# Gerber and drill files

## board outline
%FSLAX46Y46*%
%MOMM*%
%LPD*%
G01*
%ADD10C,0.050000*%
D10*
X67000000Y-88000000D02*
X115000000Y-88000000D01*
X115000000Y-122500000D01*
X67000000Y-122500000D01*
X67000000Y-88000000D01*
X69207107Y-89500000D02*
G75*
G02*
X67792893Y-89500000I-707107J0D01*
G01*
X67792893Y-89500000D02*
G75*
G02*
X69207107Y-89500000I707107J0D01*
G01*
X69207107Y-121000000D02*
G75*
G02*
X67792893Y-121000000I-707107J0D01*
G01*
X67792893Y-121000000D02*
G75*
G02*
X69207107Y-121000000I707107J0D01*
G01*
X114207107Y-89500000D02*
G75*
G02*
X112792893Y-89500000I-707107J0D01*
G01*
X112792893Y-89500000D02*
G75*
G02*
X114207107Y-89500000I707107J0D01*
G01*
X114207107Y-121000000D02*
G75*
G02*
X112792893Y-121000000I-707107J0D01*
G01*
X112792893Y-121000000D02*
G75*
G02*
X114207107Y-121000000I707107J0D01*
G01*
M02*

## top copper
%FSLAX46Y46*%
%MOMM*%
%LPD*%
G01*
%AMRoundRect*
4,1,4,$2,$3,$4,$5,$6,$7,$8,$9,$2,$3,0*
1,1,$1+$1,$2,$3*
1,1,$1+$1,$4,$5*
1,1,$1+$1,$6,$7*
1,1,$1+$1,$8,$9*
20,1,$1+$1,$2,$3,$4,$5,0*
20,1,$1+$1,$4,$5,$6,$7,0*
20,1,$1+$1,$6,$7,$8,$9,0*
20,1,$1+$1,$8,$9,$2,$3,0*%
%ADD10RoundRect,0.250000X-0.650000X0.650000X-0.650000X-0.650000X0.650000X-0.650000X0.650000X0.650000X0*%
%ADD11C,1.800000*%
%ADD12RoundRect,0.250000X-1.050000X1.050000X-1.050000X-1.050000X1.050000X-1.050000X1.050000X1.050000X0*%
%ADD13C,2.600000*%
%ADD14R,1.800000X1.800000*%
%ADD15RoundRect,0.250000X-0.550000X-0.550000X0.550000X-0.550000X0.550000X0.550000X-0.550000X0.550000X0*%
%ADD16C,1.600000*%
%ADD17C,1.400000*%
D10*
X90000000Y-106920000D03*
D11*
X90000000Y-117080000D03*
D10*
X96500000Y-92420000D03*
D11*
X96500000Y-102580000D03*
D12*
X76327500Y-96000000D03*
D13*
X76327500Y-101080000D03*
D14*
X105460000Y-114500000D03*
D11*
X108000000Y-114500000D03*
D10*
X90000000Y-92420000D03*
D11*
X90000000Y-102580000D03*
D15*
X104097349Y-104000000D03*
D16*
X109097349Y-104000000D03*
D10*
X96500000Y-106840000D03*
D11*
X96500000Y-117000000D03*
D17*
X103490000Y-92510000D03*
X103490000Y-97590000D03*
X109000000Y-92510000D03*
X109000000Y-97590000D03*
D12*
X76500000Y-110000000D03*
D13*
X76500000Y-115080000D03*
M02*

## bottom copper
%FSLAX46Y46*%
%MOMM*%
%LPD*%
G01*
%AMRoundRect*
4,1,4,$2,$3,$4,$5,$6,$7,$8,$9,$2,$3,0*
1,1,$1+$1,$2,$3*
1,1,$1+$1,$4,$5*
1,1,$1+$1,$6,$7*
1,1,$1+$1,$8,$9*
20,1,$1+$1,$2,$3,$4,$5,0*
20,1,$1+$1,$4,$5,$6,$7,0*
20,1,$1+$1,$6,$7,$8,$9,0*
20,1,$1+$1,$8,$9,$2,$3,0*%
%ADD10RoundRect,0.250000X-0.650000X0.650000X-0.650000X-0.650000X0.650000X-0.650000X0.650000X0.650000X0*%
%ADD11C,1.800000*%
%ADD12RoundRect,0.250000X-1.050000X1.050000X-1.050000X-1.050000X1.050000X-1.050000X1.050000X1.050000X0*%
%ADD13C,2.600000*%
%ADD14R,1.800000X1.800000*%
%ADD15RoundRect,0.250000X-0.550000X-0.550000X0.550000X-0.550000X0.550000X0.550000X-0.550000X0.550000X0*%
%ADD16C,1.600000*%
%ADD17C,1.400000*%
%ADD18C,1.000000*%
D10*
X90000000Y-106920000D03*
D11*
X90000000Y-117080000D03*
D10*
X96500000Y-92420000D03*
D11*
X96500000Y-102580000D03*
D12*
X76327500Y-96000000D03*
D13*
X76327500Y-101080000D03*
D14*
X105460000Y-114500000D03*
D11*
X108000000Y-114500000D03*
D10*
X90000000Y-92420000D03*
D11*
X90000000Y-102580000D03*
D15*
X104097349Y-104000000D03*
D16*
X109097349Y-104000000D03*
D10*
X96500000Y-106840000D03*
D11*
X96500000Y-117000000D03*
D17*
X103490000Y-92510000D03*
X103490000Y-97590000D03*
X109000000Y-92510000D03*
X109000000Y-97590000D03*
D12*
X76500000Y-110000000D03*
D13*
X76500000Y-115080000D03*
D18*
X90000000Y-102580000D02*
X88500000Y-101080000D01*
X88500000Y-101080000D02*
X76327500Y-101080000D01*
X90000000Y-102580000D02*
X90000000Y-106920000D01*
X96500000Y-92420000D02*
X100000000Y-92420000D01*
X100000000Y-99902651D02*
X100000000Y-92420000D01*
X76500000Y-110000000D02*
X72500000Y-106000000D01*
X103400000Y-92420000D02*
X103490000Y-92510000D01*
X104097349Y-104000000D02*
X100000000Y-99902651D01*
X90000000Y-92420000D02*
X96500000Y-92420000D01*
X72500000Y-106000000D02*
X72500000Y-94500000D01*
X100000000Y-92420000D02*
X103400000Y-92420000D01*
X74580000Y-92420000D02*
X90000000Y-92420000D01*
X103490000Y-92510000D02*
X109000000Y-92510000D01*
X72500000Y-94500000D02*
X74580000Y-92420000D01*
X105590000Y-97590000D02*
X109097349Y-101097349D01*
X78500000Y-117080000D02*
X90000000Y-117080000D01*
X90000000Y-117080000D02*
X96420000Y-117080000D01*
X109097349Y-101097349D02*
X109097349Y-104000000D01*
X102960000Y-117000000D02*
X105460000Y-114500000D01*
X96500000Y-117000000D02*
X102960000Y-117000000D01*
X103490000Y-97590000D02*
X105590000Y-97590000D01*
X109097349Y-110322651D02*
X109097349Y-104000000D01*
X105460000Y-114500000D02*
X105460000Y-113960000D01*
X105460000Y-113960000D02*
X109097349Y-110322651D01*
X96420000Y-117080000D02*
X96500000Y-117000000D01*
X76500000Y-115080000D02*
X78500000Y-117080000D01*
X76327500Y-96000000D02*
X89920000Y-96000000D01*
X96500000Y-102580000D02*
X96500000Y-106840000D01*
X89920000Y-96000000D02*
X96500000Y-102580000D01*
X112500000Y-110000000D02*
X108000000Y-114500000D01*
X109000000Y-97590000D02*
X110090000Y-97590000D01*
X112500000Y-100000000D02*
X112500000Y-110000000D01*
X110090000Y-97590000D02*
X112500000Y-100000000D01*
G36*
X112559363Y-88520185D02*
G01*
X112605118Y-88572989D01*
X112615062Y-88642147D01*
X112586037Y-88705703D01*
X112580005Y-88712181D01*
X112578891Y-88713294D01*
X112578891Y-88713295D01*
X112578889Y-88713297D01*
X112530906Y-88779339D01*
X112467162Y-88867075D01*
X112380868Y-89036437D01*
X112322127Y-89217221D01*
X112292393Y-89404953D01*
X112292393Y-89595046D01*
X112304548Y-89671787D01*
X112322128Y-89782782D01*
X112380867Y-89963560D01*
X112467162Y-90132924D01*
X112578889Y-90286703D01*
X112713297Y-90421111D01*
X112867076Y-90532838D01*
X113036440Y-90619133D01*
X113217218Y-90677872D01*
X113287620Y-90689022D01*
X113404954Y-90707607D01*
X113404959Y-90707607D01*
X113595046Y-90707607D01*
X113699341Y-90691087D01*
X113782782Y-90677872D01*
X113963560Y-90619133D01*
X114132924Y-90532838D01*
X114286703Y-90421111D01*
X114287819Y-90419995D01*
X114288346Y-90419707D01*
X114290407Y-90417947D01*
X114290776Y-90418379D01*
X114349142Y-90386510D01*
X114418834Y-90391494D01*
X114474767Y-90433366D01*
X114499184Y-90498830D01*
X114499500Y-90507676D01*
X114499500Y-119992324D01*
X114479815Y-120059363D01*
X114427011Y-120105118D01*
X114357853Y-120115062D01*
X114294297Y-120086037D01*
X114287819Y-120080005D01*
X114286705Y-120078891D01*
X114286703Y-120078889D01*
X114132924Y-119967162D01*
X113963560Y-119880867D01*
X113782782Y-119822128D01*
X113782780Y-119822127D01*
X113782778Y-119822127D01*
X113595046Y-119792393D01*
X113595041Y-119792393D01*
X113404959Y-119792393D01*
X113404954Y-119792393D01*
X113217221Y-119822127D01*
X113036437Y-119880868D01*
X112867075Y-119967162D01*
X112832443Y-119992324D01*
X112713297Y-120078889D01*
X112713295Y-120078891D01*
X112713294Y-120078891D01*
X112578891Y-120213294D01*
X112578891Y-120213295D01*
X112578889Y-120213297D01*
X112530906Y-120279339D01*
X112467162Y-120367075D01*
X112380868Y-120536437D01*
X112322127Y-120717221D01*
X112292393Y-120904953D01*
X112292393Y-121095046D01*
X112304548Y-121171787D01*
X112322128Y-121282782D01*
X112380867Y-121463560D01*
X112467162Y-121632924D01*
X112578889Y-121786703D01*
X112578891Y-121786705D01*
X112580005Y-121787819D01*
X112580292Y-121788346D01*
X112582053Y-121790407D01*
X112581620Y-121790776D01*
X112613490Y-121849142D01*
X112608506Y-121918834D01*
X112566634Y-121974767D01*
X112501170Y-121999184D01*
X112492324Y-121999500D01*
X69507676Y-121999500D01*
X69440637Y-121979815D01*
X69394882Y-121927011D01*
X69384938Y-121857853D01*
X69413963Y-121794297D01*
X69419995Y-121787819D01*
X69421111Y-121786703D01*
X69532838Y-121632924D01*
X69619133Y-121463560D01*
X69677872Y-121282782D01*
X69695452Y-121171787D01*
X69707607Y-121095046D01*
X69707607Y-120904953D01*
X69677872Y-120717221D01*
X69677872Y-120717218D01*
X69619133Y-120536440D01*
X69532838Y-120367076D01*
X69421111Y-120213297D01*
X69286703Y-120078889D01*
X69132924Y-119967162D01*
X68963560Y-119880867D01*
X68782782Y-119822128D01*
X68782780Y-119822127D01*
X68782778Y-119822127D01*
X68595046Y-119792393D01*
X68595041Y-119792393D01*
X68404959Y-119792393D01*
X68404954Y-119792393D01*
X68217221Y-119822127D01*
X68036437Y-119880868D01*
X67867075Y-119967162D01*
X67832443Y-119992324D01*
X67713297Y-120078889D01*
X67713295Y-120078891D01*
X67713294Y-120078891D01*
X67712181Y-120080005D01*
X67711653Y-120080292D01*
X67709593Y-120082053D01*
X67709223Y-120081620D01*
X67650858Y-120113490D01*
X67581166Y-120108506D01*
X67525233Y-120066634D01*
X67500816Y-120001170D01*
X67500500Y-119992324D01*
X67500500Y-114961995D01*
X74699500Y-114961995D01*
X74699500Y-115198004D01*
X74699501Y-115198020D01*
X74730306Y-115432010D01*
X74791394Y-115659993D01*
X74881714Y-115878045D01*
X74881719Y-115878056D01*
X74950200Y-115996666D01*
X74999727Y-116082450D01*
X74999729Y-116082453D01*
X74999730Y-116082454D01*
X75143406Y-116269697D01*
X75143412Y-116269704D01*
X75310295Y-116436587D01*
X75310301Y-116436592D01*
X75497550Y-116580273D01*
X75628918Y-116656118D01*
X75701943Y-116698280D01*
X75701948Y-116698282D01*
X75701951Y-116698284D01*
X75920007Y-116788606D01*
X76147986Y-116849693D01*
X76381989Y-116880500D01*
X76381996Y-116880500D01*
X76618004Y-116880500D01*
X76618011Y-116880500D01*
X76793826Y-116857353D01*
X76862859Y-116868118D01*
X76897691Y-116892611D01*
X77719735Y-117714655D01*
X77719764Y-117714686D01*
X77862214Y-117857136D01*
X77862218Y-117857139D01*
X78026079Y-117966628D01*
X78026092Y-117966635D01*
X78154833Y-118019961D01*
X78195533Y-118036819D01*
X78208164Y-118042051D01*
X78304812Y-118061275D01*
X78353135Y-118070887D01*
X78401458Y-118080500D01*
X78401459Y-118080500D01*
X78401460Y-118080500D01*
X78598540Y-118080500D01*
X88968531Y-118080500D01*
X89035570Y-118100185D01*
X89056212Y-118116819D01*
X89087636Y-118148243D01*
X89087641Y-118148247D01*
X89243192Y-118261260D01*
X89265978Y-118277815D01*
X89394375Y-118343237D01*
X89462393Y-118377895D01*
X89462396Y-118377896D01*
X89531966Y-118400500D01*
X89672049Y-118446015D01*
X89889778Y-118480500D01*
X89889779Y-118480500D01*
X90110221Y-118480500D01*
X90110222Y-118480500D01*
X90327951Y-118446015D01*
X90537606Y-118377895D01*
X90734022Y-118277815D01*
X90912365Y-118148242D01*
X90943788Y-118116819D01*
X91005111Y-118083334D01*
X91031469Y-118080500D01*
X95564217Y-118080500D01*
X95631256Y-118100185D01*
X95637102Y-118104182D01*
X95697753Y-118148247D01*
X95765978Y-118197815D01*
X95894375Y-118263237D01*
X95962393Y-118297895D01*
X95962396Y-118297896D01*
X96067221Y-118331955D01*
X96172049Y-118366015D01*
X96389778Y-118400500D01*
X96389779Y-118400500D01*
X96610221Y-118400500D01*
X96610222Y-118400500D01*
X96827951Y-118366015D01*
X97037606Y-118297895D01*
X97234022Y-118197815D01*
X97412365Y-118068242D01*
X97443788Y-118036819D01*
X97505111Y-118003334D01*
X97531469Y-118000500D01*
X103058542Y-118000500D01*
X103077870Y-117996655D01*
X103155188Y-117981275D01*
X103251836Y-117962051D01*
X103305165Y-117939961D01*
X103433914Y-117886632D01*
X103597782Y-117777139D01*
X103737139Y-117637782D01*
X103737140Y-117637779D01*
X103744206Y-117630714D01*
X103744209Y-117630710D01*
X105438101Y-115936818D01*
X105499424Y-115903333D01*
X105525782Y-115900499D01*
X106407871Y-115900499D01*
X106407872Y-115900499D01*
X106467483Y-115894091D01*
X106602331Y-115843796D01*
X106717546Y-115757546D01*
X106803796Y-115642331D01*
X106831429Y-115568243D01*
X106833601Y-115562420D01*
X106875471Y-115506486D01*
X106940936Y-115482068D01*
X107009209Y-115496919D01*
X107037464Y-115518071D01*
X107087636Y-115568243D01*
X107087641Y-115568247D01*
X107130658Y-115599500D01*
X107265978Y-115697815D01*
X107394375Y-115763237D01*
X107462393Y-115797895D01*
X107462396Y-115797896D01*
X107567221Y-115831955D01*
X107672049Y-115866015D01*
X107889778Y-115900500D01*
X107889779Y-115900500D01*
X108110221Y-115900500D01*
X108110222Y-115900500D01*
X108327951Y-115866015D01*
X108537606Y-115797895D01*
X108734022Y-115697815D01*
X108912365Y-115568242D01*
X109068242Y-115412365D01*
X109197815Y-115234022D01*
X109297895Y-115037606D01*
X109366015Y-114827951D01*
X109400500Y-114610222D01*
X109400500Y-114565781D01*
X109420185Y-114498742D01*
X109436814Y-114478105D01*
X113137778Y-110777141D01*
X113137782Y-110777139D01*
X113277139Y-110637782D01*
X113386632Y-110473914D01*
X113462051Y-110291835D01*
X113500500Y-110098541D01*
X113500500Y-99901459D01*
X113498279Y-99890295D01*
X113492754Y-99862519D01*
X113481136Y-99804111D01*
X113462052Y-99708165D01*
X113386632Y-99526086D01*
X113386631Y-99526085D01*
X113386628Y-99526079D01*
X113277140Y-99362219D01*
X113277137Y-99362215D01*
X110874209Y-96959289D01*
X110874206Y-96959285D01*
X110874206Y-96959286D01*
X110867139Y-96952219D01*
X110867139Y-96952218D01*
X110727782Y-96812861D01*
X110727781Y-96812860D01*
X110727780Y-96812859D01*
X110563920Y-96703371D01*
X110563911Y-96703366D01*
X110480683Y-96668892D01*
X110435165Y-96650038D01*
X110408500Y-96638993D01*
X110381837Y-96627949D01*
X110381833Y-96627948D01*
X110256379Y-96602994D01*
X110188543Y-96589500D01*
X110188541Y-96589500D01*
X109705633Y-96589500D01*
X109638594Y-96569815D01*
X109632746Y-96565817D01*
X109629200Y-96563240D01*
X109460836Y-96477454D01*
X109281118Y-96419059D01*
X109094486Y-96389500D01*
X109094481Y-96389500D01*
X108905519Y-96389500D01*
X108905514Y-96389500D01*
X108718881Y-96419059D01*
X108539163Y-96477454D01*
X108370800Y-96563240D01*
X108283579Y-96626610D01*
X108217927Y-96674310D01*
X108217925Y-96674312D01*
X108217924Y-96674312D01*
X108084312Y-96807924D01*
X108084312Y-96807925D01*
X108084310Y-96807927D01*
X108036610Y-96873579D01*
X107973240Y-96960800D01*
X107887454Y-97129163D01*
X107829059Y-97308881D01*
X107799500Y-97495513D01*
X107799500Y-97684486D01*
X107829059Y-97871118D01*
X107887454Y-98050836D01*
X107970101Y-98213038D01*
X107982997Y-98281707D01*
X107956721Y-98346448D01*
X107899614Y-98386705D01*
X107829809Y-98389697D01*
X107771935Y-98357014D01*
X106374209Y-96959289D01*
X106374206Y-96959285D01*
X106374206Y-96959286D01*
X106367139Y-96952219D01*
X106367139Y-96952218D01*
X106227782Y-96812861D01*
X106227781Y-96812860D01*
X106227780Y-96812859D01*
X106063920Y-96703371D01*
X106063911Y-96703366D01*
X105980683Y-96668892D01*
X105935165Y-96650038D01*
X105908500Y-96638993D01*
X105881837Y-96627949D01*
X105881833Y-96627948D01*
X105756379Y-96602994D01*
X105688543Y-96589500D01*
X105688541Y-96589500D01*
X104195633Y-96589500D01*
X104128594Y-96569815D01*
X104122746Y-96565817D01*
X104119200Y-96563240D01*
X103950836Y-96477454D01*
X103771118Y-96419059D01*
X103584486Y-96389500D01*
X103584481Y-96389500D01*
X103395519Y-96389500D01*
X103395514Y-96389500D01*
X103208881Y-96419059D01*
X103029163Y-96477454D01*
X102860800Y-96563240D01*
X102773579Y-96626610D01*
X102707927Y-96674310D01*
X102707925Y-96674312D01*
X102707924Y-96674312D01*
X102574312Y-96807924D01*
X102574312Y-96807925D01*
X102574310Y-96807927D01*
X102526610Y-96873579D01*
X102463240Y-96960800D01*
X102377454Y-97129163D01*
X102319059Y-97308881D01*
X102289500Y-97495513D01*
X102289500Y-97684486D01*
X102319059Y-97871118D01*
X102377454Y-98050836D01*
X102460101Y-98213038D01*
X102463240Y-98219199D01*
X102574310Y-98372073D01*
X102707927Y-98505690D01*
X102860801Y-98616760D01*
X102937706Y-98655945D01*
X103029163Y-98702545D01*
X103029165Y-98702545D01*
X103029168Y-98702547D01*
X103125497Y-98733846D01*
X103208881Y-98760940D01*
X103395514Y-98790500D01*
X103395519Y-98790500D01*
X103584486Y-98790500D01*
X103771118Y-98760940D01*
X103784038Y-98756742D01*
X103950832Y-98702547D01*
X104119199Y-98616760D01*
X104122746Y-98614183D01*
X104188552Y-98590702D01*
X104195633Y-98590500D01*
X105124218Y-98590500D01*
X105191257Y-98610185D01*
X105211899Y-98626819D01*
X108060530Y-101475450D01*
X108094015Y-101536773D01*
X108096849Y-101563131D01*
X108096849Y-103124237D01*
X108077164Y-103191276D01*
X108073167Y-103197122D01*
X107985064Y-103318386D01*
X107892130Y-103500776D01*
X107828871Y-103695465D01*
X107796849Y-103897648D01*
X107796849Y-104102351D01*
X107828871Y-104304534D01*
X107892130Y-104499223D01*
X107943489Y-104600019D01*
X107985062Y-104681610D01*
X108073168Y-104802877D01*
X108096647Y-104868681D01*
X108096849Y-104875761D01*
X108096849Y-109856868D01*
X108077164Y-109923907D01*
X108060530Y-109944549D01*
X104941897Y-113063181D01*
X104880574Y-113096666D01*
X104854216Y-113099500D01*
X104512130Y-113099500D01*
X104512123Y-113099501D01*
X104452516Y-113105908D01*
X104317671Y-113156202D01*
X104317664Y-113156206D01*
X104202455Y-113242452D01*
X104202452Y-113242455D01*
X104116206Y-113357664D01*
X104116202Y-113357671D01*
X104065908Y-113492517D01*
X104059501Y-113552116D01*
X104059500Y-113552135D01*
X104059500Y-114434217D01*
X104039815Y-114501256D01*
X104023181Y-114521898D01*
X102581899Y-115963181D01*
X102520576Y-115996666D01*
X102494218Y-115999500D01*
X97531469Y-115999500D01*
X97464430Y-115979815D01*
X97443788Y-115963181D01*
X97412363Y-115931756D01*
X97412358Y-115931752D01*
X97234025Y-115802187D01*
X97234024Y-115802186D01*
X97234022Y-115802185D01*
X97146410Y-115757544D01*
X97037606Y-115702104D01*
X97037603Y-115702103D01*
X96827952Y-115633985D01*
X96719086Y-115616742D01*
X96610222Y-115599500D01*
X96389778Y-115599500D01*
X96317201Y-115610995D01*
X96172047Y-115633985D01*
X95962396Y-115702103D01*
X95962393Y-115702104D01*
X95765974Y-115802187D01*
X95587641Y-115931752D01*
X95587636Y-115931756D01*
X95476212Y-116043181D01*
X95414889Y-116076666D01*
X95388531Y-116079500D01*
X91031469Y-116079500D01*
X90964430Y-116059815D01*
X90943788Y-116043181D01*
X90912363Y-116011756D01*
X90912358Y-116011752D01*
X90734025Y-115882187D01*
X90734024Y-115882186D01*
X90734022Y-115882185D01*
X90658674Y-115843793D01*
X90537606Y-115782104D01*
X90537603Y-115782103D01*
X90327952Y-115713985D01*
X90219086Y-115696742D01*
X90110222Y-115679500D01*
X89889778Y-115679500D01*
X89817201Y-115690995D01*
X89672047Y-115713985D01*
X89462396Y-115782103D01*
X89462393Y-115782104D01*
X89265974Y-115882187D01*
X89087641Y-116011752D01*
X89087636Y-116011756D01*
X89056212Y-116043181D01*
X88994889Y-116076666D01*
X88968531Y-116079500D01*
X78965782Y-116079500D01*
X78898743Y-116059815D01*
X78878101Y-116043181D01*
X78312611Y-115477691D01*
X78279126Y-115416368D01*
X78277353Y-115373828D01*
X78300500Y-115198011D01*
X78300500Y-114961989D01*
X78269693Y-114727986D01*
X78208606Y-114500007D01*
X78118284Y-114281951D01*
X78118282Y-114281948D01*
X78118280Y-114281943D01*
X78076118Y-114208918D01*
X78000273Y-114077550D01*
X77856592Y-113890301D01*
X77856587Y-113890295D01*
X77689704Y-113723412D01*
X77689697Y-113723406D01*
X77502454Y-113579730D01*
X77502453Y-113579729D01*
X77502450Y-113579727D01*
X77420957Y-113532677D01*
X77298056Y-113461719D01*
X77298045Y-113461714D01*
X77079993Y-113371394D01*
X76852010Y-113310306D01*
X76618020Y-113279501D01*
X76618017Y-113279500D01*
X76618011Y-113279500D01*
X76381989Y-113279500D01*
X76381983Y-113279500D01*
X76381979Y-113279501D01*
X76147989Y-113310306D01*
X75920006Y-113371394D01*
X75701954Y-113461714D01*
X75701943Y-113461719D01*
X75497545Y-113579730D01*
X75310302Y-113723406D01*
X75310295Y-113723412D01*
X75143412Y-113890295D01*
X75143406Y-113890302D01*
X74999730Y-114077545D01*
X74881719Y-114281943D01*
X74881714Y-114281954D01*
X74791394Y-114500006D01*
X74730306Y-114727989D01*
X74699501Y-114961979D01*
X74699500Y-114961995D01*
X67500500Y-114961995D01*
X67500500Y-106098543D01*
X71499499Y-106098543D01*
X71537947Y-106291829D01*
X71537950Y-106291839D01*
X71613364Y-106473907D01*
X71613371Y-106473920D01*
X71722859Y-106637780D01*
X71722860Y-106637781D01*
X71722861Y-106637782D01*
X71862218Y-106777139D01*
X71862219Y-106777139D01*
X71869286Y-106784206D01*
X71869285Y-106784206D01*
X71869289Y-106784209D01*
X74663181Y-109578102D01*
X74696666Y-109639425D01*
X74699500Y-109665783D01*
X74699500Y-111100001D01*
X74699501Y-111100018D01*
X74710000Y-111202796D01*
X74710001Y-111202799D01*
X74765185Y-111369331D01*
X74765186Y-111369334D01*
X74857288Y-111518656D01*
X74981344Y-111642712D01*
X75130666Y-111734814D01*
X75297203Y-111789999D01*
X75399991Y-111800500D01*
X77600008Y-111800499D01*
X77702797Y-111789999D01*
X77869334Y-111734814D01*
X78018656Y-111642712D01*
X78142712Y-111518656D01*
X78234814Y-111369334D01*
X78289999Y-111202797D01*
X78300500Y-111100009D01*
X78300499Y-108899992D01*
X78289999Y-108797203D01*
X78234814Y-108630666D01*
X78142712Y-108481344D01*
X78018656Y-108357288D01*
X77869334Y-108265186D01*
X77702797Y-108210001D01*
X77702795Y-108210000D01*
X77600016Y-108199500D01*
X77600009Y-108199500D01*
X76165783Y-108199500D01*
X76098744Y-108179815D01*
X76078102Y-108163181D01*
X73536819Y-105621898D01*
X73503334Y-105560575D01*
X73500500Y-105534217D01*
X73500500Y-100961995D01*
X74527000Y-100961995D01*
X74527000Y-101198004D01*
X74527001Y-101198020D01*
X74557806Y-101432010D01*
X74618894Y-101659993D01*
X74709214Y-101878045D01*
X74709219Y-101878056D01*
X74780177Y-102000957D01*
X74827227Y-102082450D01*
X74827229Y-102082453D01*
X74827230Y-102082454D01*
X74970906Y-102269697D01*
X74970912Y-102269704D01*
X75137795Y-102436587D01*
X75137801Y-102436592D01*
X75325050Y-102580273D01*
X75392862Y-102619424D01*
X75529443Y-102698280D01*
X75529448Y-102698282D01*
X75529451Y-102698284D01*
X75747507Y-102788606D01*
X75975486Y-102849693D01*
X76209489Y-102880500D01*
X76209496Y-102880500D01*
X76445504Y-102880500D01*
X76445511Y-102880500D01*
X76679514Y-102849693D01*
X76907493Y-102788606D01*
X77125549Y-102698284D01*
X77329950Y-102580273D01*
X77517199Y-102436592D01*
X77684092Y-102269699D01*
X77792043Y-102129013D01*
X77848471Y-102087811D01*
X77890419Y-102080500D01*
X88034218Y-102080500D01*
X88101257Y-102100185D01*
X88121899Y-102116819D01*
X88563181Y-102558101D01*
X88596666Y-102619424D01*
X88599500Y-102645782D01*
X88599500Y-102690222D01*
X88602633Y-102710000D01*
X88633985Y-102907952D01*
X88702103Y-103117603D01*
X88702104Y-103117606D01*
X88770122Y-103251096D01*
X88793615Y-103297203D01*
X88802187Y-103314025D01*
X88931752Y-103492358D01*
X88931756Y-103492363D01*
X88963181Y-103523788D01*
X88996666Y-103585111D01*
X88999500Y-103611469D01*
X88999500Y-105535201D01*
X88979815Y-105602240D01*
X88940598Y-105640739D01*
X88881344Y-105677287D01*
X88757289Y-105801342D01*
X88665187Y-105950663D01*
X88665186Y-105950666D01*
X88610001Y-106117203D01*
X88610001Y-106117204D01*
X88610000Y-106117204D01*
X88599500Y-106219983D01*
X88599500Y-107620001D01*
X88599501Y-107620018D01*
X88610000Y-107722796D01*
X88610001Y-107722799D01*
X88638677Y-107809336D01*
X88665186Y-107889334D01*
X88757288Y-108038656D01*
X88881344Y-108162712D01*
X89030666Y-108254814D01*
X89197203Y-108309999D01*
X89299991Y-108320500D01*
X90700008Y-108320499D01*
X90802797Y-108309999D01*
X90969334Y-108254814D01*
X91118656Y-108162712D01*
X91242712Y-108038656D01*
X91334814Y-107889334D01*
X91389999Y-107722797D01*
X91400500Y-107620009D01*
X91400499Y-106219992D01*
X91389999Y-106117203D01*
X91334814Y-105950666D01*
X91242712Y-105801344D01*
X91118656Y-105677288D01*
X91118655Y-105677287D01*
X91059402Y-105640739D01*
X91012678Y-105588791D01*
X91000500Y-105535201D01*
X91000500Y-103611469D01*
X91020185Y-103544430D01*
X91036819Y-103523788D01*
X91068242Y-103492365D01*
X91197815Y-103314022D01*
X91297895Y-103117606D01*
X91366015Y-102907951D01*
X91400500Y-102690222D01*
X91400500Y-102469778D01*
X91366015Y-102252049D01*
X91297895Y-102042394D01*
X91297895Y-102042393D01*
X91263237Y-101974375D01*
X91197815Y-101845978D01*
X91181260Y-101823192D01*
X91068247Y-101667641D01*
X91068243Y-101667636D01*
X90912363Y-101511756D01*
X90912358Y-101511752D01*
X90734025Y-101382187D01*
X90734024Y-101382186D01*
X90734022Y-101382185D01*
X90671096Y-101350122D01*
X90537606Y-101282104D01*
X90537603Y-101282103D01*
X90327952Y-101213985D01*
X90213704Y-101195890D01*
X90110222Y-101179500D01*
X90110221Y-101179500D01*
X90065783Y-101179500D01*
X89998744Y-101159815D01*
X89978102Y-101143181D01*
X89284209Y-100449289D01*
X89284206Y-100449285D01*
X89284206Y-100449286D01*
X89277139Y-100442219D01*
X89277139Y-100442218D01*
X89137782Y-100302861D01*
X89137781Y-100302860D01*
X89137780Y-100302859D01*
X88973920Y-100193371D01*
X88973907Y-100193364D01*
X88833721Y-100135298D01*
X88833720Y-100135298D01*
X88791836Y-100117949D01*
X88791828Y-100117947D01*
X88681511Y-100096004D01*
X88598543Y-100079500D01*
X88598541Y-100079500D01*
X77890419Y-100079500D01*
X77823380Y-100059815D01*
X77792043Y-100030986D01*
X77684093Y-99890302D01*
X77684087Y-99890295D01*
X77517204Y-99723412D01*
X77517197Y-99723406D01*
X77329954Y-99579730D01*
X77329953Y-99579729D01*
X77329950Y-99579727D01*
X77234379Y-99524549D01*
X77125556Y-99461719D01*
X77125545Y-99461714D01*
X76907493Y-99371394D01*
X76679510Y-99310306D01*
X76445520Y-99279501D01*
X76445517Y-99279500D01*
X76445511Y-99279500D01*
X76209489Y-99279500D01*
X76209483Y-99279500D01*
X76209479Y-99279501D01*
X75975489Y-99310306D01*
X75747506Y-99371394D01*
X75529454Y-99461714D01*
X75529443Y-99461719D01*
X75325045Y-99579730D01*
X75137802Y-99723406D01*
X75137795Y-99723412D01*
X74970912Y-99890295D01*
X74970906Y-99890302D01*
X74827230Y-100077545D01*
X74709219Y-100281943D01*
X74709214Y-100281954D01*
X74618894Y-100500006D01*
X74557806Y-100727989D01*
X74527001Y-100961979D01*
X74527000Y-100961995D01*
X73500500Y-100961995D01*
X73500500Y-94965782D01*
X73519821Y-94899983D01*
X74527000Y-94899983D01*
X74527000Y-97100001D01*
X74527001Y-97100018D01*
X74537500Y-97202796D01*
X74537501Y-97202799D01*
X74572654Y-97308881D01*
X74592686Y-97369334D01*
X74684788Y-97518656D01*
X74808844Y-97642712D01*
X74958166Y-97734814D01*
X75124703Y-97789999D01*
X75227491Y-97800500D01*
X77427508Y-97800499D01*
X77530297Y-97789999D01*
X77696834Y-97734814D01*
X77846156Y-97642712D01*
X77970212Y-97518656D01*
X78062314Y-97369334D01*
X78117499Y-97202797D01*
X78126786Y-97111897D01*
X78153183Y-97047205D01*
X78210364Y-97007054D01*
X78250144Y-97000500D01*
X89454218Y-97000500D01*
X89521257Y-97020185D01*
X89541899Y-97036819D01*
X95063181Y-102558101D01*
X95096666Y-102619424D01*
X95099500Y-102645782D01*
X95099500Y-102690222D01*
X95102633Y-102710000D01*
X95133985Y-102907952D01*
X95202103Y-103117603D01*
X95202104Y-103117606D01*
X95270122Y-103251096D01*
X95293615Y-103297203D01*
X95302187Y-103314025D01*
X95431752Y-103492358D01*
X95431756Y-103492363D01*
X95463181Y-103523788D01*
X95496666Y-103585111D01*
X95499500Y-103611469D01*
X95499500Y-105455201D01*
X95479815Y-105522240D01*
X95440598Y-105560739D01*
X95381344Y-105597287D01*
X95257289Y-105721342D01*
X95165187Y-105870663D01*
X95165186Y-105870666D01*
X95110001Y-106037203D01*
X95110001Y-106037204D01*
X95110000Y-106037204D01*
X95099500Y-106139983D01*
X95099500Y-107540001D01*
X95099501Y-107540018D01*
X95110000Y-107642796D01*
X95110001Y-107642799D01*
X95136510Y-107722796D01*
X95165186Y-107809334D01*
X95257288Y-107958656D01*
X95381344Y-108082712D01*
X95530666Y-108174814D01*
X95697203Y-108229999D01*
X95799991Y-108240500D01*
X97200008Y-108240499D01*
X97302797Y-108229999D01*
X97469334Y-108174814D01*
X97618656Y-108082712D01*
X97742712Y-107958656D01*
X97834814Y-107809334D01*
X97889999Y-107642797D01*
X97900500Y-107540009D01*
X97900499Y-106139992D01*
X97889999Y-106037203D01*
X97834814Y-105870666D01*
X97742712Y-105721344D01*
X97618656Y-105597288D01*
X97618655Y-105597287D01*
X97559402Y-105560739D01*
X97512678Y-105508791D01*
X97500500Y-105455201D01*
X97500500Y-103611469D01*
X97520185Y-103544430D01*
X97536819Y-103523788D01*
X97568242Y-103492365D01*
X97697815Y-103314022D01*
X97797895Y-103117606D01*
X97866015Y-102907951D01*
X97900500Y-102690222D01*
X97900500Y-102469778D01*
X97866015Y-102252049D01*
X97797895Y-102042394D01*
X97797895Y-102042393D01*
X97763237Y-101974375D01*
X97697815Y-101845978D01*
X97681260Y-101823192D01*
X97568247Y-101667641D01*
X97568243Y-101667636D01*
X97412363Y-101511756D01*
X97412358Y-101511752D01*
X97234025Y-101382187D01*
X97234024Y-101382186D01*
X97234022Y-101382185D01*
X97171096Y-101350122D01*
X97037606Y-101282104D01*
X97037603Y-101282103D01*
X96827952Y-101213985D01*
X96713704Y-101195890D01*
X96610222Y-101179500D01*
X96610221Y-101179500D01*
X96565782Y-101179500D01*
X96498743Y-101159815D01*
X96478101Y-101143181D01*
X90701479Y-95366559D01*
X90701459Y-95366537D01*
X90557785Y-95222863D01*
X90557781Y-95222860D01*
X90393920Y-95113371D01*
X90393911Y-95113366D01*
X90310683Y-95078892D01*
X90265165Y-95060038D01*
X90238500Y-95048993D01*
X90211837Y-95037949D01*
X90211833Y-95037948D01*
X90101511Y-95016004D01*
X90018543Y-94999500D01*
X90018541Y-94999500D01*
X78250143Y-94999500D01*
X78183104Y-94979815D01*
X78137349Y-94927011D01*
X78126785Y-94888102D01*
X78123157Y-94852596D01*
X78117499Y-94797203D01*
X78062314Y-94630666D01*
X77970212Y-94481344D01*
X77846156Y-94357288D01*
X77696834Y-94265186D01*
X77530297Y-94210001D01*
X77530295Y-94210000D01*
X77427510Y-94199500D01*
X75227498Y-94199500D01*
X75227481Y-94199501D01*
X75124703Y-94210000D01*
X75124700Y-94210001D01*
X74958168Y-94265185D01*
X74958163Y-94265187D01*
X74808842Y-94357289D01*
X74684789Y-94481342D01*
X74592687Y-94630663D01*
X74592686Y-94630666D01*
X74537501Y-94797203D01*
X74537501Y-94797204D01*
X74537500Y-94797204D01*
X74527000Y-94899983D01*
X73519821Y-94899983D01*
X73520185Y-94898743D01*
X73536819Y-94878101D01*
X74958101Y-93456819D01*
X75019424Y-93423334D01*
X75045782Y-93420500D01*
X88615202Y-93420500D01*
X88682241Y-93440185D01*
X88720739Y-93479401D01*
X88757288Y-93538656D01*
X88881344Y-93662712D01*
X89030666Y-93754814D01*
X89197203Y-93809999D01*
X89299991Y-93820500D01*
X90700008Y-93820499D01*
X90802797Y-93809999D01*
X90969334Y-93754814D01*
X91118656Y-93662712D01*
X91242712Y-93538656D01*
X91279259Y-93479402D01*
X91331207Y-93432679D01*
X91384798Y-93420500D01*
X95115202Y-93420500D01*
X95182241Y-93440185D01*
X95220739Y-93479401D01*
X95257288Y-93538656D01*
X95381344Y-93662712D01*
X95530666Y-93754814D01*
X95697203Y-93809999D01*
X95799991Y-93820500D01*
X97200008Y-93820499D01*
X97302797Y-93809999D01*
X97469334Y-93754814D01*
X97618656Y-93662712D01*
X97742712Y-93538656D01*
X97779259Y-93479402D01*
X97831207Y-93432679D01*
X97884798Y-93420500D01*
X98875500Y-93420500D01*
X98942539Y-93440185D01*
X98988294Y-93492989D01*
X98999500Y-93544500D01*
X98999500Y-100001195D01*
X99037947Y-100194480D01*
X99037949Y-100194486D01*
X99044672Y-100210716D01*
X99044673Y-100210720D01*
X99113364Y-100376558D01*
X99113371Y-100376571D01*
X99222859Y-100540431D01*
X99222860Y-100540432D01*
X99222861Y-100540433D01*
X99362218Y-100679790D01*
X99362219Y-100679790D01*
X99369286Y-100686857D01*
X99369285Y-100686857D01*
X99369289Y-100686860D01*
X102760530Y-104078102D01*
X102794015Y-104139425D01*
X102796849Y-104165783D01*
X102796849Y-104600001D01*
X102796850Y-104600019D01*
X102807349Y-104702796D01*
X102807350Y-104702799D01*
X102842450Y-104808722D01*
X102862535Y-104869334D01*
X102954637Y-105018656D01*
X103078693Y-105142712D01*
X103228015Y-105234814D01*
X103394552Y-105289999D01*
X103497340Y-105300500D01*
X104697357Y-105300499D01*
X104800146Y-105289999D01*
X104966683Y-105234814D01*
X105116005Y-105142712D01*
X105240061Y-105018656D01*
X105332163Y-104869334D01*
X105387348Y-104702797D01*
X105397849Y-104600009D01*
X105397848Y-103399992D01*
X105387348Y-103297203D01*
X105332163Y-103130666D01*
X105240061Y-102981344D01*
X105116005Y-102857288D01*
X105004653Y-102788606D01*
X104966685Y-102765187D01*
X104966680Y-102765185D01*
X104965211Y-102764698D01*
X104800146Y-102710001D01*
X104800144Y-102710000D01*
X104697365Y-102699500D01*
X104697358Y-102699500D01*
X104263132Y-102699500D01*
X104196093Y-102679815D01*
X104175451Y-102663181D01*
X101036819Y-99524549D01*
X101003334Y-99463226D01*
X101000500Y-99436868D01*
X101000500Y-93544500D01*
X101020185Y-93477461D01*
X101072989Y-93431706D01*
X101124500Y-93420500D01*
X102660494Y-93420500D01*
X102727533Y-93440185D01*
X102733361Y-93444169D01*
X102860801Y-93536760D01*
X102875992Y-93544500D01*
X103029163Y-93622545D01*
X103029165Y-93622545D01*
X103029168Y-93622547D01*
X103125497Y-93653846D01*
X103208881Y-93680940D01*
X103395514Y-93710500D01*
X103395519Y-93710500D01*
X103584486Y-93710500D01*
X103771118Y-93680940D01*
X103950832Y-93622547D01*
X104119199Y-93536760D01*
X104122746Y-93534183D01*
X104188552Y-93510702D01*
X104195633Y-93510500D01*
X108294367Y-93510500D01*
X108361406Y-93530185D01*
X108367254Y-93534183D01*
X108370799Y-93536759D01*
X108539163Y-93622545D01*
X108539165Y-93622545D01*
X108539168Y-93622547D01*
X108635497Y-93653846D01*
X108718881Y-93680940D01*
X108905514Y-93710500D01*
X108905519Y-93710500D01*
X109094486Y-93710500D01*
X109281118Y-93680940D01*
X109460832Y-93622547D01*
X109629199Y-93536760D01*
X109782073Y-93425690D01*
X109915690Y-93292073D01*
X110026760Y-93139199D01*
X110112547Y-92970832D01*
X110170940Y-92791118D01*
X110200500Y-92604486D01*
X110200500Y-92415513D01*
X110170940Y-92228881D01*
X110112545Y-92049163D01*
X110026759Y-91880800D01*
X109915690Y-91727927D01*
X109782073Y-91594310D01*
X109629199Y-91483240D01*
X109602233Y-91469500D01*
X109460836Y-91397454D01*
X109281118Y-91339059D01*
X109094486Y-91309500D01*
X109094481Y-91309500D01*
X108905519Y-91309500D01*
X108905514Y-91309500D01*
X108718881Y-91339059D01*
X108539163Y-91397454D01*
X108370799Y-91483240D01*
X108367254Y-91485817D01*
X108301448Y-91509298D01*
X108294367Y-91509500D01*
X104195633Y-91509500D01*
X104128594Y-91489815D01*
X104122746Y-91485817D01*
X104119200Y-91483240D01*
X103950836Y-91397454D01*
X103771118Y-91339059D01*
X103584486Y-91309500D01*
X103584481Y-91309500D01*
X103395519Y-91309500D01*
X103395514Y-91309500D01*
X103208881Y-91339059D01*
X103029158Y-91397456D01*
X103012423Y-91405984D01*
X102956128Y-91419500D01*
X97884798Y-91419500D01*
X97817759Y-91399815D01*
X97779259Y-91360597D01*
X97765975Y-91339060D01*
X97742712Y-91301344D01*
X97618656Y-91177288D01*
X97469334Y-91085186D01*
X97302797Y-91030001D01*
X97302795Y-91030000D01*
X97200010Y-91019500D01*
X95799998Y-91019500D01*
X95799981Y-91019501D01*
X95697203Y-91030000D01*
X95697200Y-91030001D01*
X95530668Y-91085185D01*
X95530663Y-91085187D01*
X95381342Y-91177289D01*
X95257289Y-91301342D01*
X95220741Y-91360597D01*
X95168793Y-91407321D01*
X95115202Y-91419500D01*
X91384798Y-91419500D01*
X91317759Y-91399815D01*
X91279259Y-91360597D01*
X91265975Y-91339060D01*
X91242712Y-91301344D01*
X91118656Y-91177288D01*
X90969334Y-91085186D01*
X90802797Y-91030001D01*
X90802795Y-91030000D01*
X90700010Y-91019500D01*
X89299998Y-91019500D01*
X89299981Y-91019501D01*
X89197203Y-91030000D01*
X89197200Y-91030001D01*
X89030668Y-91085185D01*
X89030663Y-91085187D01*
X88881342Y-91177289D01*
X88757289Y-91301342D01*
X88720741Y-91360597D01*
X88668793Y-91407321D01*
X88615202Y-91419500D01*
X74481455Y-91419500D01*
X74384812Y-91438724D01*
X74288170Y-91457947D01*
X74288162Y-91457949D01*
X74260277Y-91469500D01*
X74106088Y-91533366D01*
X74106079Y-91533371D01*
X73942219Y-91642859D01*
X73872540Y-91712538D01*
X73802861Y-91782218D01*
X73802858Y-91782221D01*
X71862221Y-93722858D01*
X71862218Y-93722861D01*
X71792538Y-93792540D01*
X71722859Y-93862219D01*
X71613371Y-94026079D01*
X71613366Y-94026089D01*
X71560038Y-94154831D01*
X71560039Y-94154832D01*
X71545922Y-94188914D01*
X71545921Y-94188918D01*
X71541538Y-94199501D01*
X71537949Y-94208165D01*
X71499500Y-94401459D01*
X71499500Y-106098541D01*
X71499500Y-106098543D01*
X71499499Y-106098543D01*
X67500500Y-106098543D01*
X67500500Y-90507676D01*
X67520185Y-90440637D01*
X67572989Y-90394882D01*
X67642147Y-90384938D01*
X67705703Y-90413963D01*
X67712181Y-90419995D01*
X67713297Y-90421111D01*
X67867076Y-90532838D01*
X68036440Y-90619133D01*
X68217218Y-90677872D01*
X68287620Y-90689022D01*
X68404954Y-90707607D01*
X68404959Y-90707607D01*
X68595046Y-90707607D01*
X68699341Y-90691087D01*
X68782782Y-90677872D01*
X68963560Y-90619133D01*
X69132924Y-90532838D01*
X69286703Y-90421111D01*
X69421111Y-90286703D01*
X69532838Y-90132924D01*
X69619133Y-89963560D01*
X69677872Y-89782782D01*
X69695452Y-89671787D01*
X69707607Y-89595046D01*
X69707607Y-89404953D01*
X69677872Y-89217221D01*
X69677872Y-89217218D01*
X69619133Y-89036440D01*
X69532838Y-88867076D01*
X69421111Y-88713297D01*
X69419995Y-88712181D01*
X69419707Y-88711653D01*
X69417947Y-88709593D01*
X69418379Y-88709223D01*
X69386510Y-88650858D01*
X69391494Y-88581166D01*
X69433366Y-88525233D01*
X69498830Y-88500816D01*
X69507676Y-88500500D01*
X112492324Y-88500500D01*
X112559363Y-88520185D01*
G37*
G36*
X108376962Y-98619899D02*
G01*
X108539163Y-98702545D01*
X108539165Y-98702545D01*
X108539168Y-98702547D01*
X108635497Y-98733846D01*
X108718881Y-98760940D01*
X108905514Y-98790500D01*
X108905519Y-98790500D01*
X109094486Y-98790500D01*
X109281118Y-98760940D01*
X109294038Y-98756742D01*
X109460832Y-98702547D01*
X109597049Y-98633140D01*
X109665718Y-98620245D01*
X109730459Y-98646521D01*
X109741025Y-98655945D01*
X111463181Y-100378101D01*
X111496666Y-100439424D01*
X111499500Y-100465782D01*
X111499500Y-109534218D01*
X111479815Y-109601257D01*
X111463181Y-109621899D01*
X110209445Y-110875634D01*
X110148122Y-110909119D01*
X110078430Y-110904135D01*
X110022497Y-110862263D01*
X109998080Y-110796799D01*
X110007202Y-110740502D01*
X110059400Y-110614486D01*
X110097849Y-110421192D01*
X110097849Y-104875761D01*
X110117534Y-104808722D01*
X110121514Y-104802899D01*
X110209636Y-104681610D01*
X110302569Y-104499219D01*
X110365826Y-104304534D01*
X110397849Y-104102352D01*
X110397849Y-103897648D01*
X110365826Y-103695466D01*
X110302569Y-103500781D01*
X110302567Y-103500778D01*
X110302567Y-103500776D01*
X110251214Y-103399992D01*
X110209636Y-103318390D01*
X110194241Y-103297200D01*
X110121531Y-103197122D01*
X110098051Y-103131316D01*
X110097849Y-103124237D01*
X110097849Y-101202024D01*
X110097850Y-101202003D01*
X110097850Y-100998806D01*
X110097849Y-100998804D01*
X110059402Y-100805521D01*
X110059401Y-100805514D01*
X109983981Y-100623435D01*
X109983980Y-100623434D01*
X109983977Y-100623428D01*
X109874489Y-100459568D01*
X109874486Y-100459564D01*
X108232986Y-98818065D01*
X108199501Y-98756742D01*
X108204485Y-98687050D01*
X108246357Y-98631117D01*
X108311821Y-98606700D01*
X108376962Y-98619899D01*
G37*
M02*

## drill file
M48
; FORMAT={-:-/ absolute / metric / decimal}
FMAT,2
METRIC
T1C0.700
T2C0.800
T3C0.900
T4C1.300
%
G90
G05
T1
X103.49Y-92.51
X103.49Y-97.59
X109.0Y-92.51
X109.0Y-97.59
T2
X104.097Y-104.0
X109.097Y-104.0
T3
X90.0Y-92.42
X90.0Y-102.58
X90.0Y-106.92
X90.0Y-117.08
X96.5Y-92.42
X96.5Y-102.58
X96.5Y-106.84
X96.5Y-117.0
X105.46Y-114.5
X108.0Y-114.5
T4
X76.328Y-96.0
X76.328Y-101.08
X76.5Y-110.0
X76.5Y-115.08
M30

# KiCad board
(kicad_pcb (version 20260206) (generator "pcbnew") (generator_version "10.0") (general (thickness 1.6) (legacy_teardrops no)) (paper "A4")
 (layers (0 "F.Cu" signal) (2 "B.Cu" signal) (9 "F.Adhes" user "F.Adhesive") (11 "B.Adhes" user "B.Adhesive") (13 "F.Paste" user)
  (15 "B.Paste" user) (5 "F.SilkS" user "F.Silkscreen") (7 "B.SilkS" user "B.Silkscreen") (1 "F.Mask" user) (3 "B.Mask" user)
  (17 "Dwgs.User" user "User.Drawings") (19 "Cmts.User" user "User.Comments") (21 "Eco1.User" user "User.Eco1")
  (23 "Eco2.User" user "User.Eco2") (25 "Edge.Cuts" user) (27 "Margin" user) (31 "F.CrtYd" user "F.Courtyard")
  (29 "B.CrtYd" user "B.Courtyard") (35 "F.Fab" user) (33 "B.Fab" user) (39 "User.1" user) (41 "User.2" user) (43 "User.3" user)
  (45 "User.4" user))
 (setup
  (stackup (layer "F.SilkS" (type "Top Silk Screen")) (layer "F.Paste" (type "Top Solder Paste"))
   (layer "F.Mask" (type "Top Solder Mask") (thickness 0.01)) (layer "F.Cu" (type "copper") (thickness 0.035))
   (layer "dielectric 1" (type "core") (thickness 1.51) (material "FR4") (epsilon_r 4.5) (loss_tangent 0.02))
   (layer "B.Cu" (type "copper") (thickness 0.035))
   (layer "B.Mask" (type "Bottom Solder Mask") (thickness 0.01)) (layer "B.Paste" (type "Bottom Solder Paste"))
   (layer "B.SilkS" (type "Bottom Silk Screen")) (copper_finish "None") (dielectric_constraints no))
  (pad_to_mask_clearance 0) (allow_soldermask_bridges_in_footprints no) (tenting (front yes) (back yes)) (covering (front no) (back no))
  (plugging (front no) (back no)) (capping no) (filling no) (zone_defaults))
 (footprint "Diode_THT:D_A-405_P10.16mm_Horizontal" (layer "F.Cu") (at 90 106.92 -90)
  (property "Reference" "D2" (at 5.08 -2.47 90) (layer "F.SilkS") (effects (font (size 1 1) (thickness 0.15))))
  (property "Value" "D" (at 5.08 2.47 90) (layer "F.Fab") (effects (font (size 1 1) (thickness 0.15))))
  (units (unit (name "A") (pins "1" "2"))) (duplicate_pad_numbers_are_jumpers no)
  (pad "1" thru_hole roundrect (at 0 0 270) (size 1.8 1.8) (drill 0.9) (layers "*.Cu" "*.Mask") (remove_unused_layers no)
   (roundrect_rratio 0.138889) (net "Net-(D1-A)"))
  (pad "2" thru_hole circle (at 10.16 0 270) (size 1.8 1.8) (drill 0.9) (layers "*.Cu" "*.Mask") (remove_unused_layers no)
   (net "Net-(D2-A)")))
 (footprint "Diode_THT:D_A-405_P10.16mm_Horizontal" (layer "F.Cu") (at 96.5 92.42 -90)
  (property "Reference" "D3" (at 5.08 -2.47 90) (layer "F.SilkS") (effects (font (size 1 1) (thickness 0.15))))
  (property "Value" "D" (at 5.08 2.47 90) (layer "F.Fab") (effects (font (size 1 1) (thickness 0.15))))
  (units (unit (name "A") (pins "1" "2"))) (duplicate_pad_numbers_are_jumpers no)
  (pad "1" thru_hole roundrect (at 0 0 270) (size 1.8 1.8) (drill 0.9) (layers "*.Cu" "*.Mask") (remove_unused_layers no)
   (roundrect_rratio 0.138889) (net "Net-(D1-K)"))
  (pad "2" thru_hole circle (at 10.16 0 270) (size 1.8 1.8) (drill 0.9) (layers "*.Cu" "*.Mask") (remove_unused_layers no)
   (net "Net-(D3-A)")))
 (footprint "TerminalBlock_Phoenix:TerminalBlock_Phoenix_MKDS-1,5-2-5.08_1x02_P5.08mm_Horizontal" (layer "F.Cu") (at 76.3275 96 -90)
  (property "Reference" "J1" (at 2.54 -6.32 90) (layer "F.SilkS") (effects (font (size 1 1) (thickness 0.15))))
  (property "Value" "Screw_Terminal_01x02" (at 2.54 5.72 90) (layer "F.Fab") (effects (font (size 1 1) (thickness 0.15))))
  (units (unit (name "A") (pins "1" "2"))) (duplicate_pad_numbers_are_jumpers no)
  (pad "1" thru_hole roundrect (at 0 0 270) (size 2.6 2.6) (drill 1.3) (layers "*.Cu" "*.Mask") (remove_unused_layers no)
   (roundrect_rratio 0.096154) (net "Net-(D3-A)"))
  (pad "2" thru_hole circle (at 5.08 0 270) (size 2.6 2.6) (drill 1.3) (layers "*.Cu" "*.Mask") (remove_unused_layers no) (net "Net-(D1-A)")))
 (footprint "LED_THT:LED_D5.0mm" (layer "F.Cu") (at 105.46 114.5)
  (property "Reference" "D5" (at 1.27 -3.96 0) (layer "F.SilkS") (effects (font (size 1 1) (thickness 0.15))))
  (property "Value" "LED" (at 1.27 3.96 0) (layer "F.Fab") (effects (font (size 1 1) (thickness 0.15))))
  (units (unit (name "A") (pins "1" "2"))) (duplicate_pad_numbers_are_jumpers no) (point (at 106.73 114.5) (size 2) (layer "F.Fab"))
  (pad "1" thru_hole rect (at 0 0) (size 1.8 1.8) (drill 0.9) (layers "*.Cu" "*.Mask") (remove_unused_layers no) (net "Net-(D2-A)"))
  (pad "2" thru_hole circle (at 2.54 0) (size 1.8 1.8) (drill 0.9) (layers "*.Cu" "*.Mask") (remove_unused_layers no) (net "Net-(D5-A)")))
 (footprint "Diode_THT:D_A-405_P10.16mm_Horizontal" (layer "F.Cu") (at 90 92.42 -90)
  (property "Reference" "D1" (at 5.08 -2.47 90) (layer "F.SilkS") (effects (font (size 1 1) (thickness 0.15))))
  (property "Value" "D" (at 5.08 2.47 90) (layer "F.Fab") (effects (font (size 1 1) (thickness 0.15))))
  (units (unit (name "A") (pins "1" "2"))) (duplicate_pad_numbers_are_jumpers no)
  (pad "1" thru_hole roundrect (at 0 0 270) (size 1.8 1.8) (drill 0.9) (layers "*.Cu" "*.Mask") (remove_unused_layers no)
   (roundrect_rratio 0.138889) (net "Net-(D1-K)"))
  (pad "2" thru_hole circle (at 10.16 0 270) (size 1.8 1.8) (drill 0.9) (layers "*.Cu" "*.Mask") (remove_unused_layers no)
   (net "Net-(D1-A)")))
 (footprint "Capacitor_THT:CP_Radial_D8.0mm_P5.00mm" (layer "F.Cu") (at 104.097349 104)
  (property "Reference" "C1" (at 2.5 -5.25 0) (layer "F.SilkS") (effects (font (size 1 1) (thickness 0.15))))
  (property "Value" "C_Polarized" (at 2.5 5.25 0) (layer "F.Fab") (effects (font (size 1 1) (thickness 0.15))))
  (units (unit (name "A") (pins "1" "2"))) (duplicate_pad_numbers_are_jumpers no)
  (pad "1" thru_hole roundrect (at 0 0) (size 1.6 1.6) (drill 0.8) (layers "*.Cu" "*.Mask") (remove_unused_layers no)
   (roundrect_rratio 0.15625) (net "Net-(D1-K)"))
  (pad "2" thru_hole circle (at 5 0) (size 1.6 1.6) (drill 0.8) (layers "*.Cu" "*.Mask") (remove_unused_layers no) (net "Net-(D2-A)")))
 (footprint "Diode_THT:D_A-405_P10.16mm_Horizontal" (layer "F.Cu") (at 96.5 106.84 -90)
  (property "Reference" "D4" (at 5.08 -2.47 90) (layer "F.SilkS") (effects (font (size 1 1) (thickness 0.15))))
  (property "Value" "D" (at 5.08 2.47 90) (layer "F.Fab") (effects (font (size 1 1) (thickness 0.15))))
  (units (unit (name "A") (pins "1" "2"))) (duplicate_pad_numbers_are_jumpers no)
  (pad "1" thru_hole roundrect (at 0 0 270) (size 1.8 1.8) (drill 0.9) (layers "*.Cu" "*.Mask") (remove_unused_layers no)
   (roundrect_rratio 0.138889) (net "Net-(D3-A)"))
  (pad "2" thru_hole circle (at 10.16 0 270) (size 1.8 1.8) (drill 0.9) (layers "*.Cu" "*.Mask") (remove_unused_layers no)
   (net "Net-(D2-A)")))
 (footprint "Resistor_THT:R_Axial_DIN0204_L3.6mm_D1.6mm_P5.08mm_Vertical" (layer "F.Cu") (at 103.49 92.51 -90)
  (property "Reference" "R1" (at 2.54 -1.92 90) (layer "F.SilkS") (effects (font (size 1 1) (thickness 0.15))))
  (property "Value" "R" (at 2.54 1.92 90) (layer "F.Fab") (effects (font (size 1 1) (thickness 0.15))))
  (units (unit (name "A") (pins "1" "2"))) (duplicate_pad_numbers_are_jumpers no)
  (pad "1" thru_hole circle (at 0 0 270) (size 1.4 1.4) (drill 0.7) (layers "*.Cu" "*.Mask") (remove_unused_layers no) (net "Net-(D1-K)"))
  (pad "2" thru_hole circle (at 5.08 0 270) (size 1.4 1.4) (drill 0.7) (layers "*.Cu" "*.Mask") (remove_unused_layers no) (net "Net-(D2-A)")))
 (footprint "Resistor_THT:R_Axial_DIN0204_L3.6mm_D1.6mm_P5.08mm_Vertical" (layer "F.Cu") (at 109 92.51 -90)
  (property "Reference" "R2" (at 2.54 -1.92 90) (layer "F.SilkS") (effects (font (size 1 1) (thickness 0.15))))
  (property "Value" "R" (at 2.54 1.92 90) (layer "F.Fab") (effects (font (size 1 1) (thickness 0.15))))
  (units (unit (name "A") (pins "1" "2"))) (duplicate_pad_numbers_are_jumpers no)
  (pad "1" thru_hole circle (at 0 0 270) (size 1.4 1.4) (drill 0.7) (layers "*.Cu" "*.Mask") (remove_unused_layers no) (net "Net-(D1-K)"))
  (pad "2" thru_hole circle (at 5.08 0 270) (size 1.4 1.4) (drill 0.7) (layers "*.Cu" "*.Mask") (remove_unused_layers no) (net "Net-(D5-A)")))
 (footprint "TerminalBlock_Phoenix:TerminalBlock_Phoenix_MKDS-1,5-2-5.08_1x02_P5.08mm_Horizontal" (layer "F.Cu") (at 76.5 110 -90)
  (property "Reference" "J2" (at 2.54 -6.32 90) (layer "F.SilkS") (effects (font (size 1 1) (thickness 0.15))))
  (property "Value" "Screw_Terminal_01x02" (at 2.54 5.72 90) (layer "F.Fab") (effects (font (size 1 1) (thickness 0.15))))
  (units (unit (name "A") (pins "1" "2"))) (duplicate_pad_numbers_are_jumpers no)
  (pad "1" thru_hole roundrect (at 0 0 270) (size 2.6 2.6) (drill 1.3) (layers "*.Cu" "*.Mask") (remove_unused_layers no)
   (roundrect_rratio 0.096154) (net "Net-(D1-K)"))
  (pad "2" thru_hole circle (at 5.08 0 270) (size 2.6 2.6) (drill 1.3) (layers "*.Cu" "*.Mask") (remove_unused_layers no) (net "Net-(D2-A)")))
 (gr_rect (start 67 88) (end 115 122.5) (stroke (width 0.05) (type default)) (fill no) (layer "Edge.Cuts"))
 (gr_circle (center 68.5 89.5) (end 68 90) (stroke (width 0.05) (type default)) (fill no) (layer "Edge.Cuts"))
 (gr_circle (center 68.5 121) (end 68 121.5) (stroke (width 0.05) (type default)) (fill no) (layer "Edge.Cuts"))
 (gr_circle (center 113.5 89.5) (end 113 90) (stroke (width 0.05) (type default)) (fill no) (layer "Edge.Cuts"))
 (gr_circle (center 113.5 121) (end 113 121.5) (stroke (width 0.05) (type default)) (fill no) (layer "Edge.Cuts"))
 (segment (start 90 102.58) (end 88.5 101.08) (width 1) (layer "B.Cu") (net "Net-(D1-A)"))
 (segment (start 88.5 101.08) (end 76.3275 101.08) (width 1) (layer "B.Cu") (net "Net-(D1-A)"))
 (segment (start 90 102.58) (end 90 106.92) (width 1) (layer "B.Cu") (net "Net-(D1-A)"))
 (segment (start 96.5 92.42) (end 100 92.42) (width 1) (layer "B.Cu") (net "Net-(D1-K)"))
 (segment (start 100 99.902651) (end 100 92.42) (width 1) (layer "B.Cu") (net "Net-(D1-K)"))
 (segment (start 76.5 110) (end 72.5 106) (width 1) (layer "B.Cu") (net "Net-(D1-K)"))
 (segment (start 103.4 92.42) (end 103.49 92.51) (width 1) (layer "B.Cu") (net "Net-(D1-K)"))
 (segment (start 104.097349 104) (end 100 99.902651) (width 1) (layer "B.Cu") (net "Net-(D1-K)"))
 (segment (start 90 92.42) (end 96.5 92.42) (width 1) (layer "B.Cu") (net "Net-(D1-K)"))
 (segment (start 72.5 106) (end 72.5 94.5) (width 1) (layer "B.Cu") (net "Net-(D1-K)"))
 (segment (start 100 92.42) (end 103.4 92.42) (width 1) (layer "B.Cu") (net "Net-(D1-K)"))
 (segment (start 74.58 92.42) (end 90 92.42) (width 1) (layer "B.Cu") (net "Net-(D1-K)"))
 (segment (start 103.49 92.51) (end 109 92.51) (width 1) (layer "B.Cu") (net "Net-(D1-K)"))
 (segment (start 72.5 94.5) (end 74.58 92.42) (width 1) (layer "B.Cu") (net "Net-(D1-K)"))
 (segment (start 105.59 97.59) (end 109.097349 101.097349) (width 1) (layer "B.Cu") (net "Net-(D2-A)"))
 (segment (start 78.5 117.08) (end 90 117.08) (width 1) (layer "B.Cu") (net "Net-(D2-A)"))
 (segment (start 90 117.08) (end 96.42 117.08) (width 1) (layer "B.Cu") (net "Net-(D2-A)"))
 (segment (start 109.097349 101.097349) (end 109.097349 104) (width 1) (layer "B.Cu") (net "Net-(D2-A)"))
 (segment (start 102.96 117) (end 105.46 114.5) (width 1) (layer "B.Cu") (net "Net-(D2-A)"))
 (segment (start 96.5 117) (end 102.96 117) (width 1) (layer "B.Cu") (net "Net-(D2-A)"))
 (segment (start 103.49 97.59) (end 105.59 97.59) (width 1) (layer "B.Cu") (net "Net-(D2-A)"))
 (segment (start 109.097349 110.322651) (end 109.097349 104) (width 1) (layer "B.Cu") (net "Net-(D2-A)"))
 (segment (start 105.46 114.5) (end 105.46 113.96) (width 1) (layer "B.Cu") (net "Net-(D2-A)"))
 (segment (start 105.46 113.96) (end 109.097349 110.322651) (width 1) (layer "B.Cu") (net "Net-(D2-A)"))
 (segment (start 96.42 117.08) (end 96.5 117) (width 1) (layer "B.Cu") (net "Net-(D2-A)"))
 (segment (start 76.5 115.08) (end 78.5 117.08) (width 1) (layer "B.Cu") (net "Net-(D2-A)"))
 (segment (start 76.3275 96) (end 89.92 96) (width 1) (layer "B.Cu") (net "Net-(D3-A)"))
 (segment (start 96.5 102.58) (end 96.5 106.84) (width 1) (layer "B.Cu") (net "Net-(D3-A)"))
 (segment (start 89.92 96) (end 96.5 102.58) (width 1) (layer "B.Cu") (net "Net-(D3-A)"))
 (segment (start 112.5 110) (end 108 114.5) (width 1) (layer "B.Cu") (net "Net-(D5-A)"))
 (segment (start 109 97.59) (end 110.09 97.59) (width 1) (layer "B.Cu") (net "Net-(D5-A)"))
 (segment (start 112.5 100) (end 112.5 110) (width 1) (layer "B.Cu") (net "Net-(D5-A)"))
 (segment (start 110.09 97.59) (end 112.5 100) (width 1) (layer "B.Cu") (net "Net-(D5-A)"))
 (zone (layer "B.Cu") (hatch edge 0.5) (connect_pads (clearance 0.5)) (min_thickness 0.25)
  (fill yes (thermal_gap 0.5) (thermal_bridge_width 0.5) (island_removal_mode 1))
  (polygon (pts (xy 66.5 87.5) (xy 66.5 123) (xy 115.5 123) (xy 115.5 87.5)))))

